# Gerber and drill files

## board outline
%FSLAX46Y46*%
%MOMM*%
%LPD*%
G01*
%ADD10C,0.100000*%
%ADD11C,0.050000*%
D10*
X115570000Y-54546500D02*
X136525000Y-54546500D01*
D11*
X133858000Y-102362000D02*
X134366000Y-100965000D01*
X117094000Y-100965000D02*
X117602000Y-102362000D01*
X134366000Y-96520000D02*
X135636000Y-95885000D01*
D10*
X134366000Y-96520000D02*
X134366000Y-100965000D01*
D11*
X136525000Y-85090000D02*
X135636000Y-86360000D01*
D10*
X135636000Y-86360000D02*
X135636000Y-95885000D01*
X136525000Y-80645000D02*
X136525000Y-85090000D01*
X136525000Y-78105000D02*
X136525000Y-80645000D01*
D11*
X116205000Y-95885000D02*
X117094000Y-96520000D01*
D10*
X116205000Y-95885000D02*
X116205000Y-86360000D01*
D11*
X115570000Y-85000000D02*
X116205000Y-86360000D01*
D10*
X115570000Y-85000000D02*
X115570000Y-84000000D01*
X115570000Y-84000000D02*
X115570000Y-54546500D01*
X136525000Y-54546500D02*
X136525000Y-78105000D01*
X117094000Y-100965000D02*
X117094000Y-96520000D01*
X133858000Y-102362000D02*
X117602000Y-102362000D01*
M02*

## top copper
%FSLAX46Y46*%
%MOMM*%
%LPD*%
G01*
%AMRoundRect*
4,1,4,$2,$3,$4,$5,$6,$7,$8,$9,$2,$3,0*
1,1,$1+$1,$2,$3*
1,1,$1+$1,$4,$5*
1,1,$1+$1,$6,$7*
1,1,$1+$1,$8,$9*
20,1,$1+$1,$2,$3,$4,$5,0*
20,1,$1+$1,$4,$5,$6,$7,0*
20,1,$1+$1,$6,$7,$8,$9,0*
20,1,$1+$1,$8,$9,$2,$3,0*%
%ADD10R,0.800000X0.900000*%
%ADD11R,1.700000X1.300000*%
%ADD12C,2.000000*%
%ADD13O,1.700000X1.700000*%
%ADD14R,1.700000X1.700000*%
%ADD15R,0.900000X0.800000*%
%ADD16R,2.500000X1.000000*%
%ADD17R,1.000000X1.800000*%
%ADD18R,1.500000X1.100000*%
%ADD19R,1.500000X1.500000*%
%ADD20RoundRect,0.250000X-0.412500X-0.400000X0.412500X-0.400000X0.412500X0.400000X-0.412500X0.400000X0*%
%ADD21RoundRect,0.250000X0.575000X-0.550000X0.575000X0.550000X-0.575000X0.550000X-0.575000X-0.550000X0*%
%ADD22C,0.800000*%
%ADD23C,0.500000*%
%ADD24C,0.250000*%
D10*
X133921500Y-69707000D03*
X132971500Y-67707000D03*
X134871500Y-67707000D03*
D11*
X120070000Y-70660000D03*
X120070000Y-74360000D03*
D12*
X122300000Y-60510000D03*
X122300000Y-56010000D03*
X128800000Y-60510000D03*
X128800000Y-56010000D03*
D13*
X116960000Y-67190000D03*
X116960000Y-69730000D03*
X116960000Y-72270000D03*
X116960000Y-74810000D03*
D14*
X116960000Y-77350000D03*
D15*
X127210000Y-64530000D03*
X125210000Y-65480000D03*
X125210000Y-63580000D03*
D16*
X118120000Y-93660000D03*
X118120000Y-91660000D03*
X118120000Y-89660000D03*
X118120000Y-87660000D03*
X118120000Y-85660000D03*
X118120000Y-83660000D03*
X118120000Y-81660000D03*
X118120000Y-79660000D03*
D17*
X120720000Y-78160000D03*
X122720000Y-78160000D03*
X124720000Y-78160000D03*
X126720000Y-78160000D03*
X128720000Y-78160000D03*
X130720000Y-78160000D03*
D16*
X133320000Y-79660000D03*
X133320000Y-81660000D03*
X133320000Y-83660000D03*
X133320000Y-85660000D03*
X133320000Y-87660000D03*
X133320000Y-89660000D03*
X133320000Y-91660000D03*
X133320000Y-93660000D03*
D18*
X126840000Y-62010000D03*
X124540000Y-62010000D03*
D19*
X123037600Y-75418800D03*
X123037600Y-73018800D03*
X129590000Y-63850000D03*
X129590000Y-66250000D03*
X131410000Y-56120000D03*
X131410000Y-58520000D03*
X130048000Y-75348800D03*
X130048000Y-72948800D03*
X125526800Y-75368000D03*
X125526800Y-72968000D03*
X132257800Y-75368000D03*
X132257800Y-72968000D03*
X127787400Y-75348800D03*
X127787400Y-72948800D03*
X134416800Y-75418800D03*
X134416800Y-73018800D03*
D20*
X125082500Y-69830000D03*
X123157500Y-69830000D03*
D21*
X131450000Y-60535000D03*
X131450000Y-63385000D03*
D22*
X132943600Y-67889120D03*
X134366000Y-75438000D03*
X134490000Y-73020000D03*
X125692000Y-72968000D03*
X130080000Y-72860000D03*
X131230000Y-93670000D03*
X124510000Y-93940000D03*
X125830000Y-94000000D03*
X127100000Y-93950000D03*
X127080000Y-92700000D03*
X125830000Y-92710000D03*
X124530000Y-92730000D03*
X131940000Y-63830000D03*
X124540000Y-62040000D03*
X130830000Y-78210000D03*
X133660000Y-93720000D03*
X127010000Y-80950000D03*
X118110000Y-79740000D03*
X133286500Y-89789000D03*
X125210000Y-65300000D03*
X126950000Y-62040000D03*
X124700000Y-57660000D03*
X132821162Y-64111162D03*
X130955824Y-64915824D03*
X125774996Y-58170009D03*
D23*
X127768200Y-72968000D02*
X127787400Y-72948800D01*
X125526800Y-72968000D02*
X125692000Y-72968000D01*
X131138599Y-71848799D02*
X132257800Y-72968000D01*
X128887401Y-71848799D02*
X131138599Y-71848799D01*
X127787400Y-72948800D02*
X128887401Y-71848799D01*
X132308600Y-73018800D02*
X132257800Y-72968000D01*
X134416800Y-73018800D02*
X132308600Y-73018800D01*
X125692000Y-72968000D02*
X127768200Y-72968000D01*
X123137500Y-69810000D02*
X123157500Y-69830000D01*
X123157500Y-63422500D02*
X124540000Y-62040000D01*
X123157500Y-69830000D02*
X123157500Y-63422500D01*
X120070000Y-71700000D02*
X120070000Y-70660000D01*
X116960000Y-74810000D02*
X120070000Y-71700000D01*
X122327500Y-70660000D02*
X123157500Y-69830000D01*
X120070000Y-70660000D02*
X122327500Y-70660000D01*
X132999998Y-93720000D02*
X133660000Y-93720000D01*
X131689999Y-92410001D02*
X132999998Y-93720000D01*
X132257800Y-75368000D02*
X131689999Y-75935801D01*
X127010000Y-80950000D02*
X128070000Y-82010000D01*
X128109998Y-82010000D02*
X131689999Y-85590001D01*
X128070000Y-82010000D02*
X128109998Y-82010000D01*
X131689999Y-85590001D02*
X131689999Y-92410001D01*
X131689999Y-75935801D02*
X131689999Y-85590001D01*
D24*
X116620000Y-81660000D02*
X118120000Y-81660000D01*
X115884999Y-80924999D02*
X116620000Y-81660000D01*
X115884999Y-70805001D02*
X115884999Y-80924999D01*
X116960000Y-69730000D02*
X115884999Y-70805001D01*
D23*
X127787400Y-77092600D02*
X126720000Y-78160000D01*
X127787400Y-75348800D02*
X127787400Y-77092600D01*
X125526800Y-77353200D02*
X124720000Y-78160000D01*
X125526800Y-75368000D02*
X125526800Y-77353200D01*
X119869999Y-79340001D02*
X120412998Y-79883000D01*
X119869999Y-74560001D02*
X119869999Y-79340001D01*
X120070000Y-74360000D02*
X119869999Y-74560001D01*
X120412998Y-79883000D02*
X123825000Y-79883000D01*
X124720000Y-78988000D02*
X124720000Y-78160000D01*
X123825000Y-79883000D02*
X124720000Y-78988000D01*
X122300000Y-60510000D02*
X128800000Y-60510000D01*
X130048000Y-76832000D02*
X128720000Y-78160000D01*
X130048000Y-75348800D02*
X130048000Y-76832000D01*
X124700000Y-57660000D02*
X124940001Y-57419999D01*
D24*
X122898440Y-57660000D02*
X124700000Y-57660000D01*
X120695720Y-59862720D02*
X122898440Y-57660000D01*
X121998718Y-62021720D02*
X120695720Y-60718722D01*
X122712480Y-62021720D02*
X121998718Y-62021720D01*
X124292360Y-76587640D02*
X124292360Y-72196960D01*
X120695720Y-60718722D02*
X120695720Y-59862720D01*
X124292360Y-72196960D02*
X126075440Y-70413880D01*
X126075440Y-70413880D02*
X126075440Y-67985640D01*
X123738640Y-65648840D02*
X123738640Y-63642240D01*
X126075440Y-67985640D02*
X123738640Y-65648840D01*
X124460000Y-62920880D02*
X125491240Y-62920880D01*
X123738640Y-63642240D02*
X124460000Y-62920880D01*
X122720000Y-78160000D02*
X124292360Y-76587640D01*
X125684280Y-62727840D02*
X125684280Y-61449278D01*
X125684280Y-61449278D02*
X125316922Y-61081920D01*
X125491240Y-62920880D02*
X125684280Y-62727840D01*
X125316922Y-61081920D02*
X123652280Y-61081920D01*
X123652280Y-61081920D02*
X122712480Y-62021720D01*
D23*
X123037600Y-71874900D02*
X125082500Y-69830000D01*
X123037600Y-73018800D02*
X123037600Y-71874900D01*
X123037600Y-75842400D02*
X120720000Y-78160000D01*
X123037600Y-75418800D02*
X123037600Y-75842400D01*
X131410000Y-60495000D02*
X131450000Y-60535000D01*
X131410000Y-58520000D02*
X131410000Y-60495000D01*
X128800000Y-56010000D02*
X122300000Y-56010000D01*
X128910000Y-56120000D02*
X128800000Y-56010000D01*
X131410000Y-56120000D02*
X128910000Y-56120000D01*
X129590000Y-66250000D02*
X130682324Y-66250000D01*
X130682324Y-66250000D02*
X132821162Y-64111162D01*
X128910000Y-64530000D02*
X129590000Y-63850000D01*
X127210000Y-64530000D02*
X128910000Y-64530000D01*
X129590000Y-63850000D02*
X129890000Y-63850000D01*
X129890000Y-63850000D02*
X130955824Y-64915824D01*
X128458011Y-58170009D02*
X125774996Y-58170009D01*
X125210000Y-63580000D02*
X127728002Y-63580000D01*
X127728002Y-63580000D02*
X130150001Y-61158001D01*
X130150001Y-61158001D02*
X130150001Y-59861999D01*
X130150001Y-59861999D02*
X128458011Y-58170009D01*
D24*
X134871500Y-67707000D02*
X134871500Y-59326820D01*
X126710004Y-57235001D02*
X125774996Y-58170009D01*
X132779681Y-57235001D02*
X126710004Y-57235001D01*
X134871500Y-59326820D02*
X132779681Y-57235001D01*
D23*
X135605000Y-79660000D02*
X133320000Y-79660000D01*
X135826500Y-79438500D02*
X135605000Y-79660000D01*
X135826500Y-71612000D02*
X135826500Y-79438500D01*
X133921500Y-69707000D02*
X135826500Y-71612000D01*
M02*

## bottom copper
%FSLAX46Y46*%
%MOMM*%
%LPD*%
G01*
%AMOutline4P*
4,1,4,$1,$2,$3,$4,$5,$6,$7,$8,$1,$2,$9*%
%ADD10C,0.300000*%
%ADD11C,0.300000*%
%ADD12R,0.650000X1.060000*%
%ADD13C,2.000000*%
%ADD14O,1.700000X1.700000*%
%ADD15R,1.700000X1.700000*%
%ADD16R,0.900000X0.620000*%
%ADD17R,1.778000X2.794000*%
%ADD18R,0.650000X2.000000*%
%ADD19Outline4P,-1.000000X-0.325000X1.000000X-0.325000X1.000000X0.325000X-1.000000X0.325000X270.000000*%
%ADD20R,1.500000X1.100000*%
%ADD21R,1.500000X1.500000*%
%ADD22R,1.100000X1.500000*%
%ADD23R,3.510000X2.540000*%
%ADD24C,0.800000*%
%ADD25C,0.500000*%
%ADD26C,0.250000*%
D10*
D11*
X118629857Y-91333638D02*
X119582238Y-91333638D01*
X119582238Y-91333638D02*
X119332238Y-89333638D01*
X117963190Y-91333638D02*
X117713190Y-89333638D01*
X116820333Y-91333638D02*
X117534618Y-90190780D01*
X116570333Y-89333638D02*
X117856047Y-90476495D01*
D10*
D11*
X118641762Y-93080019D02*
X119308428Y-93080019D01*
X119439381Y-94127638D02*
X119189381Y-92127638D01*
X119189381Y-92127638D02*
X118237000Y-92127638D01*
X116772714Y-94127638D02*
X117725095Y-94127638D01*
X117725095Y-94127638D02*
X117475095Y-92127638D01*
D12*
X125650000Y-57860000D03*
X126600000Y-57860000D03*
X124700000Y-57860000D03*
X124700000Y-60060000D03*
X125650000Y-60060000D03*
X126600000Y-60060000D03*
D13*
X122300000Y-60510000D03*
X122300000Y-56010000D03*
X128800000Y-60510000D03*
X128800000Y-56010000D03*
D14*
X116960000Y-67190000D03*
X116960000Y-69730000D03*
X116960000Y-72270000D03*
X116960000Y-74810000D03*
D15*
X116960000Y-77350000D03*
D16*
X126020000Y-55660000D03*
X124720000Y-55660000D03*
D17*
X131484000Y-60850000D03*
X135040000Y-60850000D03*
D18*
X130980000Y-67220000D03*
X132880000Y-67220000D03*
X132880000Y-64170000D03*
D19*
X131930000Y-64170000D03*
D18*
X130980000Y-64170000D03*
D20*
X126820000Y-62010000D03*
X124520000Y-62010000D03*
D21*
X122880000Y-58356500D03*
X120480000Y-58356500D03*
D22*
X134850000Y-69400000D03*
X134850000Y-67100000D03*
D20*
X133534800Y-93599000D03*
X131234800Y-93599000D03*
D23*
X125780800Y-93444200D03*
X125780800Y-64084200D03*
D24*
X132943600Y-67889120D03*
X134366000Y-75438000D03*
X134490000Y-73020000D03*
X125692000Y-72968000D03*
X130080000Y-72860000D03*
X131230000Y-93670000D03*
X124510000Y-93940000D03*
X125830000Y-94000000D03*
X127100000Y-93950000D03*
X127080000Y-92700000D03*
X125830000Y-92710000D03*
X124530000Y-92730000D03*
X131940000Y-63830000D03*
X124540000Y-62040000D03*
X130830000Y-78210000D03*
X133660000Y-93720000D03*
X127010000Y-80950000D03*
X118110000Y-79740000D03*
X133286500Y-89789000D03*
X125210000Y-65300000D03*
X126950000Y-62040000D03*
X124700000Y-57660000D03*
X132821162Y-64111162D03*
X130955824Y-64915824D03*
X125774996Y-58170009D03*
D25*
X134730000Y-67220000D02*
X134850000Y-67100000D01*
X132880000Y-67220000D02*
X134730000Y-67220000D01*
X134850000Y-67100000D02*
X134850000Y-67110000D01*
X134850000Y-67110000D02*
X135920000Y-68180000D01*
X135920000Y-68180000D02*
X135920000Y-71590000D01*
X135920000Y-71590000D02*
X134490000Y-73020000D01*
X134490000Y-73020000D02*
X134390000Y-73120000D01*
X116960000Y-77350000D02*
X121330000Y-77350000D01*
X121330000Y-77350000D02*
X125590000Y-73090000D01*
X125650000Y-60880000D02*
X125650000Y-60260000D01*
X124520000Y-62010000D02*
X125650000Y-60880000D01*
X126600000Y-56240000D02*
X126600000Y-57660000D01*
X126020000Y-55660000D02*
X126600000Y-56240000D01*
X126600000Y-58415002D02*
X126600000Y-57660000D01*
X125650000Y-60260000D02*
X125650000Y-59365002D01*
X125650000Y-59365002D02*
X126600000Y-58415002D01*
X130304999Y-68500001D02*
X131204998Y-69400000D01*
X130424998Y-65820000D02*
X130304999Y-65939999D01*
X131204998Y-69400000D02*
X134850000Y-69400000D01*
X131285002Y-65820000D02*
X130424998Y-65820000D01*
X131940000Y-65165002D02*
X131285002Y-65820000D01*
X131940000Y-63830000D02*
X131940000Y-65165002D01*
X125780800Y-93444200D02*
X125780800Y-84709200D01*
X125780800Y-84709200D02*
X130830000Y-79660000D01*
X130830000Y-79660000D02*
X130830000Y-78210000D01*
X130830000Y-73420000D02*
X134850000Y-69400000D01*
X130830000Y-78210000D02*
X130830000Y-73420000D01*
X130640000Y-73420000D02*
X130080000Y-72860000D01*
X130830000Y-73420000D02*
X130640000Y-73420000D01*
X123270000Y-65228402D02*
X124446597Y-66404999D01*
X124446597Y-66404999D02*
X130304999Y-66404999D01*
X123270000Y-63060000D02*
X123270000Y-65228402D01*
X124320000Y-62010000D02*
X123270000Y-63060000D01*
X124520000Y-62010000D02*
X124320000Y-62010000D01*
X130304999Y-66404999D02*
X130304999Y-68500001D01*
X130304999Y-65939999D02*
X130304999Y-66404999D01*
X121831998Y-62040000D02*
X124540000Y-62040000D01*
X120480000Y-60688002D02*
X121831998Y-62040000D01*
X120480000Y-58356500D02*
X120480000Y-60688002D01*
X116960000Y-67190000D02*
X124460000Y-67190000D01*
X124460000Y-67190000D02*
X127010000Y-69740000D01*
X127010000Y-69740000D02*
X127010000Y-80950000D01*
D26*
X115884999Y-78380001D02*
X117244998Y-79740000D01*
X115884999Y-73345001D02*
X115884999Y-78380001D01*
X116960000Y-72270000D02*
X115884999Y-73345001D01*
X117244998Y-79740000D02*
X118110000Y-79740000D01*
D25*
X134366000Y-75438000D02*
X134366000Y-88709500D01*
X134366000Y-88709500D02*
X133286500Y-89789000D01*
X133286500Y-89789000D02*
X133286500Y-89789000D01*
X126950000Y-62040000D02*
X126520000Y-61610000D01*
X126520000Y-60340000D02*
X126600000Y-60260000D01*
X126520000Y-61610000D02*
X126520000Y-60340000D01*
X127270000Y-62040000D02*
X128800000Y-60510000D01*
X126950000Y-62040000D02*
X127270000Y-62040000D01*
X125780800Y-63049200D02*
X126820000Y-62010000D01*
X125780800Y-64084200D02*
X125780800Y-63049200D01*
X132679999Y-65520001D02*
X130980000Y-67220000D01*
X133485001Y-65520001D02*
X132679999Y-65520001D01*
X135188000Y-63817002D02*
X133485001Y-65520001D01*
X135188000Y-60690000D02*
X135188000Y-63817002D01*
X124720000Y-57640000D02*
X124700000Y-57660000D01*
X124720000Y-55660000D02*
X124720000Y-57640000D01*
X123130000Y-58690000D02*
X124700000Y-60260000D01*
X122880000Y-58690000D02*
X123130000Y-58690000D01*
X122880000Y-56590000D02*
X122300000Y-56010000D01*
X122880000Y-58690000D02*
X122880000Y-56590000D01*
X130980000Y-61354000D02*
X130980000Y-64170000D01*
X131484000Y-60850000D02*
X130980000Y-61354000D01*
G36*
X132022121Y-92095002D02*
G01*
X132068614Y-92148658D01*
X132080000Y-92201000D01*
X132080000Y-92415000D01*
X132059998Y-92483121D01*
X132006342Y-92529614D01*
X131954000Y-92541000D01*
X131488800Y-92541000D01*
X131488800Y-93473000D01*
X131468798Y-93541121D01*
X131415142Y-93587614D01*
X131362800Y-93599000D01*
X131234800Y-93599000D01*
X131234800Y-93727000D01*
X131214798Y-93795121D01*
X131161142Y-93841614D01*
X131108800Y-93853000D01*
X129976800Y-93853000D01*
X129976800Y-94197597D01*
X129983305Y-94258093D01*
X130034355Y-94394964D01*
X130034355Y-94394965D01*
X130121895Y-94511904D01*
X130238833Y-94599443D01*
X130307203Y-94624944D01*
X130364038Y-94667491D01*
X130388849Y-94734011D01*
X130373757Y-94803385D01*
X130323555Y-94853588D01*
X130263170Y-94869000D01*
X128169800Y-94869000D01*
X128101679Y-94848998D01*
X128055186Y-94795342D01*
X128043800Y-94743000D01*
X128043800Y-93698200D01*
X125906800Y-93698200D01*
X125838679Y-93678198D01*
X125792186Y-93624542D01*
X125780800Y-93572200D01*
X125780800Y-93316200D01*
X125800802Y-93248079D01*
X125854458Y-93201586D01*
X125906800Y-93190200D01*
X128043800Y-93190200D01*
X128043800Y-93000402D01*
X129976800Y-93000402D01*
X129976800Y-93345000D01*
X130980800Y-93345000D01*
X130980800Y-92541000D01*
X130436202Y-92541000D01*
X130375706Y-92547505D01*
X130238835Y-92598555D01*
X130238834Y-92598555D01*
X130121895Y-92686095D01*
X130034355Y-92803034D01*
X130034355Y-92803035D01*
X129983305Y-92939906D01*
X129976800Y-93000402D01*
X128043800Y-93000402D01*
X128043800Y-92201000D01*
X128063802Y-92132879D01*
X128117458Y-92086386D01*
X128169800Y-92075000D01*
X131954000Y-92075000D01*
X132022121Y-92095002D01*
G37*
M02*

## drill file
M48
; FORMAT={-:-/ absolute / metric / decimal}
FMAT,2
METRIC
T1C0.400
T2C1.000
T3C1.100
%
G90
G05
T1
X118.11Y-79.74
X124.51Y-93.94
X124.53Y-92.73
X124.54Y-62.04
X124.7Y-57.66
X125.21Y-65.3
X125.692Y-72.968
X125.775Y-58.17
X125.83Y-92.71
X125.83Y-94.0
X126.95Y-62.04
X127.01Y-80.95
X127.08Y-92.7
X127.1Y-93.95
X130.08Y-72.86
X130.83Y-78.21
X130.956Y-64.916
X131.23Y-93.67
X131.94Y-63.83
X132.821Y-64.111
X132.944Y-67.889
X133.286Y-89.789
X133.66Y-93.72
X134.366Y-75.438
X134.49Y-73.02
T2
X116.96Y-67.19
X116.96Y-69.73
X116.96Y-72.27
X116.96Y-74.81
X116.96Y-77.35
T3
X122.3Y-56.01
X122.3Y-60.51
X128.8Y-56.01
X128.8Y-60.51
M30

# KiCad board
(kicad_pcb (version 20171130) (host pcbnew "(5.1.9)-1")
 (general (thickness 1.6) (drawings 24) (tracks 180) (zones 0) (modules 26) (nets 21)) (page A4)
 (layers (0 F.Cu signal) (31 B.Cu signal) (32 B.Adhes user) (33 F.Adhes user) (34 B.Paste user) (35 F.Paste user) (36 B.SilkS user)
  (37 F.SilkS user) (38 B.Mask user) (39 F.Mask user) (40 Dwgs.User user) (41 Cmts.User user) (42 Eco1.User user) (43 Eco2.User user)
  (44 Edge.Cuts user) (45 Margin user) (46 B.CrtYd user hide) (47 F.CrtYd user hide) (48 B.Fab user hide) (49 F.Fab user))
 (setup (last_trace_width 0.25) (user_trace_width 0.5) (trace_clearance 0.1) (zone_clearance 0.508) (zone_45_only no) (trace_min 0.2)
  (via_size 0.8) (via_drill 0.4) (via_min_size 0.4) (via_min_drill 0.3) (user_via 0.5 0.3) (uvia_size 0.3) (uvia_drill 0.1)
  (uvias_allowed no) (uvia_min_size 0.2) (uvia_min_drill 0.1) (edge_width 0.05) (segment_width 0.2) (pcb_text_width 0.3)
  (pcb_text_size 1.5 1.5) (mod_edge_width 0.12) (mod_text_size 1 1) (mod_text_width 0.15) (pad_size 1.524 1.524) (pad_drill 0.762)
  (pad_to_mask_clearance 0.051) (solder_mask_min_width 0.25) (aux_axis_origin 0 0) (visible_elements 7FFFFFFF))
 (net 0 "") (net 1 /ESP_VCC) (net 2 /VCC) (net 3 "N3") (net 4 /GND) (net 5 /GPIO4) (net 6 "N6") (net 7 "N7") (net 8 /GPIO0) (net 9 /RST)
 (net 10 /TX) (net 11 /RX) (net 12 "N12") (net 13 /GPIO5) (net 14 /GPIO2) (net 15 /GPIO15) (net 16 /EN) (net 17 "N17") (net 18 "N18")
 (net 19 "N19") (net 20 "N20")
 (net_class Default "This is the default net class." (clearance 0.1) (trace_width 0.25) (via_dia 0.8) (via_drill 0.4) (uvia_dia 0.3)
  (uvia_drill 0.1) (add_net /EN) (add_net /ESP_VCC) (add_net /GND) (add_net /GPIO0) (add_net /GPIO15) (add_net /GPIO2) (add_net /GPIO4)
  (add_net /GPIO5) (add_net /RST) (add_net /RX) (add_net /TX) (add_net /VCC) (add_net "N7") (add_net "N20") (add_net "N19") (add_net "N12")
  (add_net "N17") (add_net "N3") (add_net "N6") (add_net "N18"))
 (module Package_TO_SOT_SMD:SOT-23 (layer F.Cu) (at 133.9215 68.707 270)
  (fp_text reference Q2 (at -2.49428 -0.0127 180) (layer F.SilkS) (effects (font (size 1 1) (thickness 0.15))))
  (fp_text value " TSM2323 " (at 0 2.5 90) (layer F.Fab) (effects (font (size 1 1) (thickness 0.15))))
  (pad 3 smd rect (at 1 0 270) (size 0.9 0.8) (layers F.Cu F.Paste F.Mask) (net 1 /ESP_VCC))
  (pad 2 smd rect (at -1 0.95 270) (size 0.9 0.8) (layers F.Cu F.Paste F.Mask) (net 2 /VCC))
  (pad 1 smd rect (at -1 -0.95 270) (size 0.9 0.8) (layers F.Cu F.Paste F.Mask) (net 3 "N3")))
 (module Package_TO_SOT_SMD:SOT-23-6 (layer B.Cu) (at 125.65 58.96 90)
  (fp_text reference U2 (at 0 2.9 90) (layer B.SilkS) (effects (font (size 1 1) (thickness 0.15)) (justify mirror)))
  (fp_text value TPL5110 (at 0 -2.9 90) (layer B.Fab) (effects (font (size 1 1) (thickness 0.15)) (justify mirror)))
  (pad 5 smd rect (at 1.1 0 90) (size 1.06 0.65) (layers B.Cu B.Paste B.Mask) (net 3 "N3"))
  (pad 6 smd rect (at 1.1 0.95 90) (size 1.06 0.65) (layers B.Cu B.Paste B.Mask) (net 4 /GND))
  (pad 4 smd rect (at 1.1 -0.95 90) (size 1.06 0.65) (layers B.Cu B.Paste B.Mask) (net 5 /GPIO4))
  (pad 3 smd rect (at -1.1 -0.95 90) (size 1.06 0.65) (layers B.Cu B.Paste B.Mask) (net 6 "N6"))
  (pad 2 smd rect (at -1.1 0 90) (size 1.06 0.65) (layers B.Cu B.Paste B.Mask) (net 4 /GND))
  (pad 1 smd rect (at -1.1 0.95 90) (size 1.06 0.65) (layers B.Cu B.Paste B.Mask) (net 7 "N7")))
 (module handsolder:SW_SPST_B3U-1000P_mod (layer F.Cu) (at 120.07 72.51 90)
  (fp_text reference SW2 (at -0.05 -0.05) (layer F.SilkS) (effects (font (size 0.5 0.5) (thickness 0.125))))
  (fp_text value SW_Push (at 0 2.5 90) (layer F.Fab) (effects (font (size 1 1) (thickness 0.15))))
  (pad 2 smd rect (at 1.85 0 90) (size 1.3 1.7) (layers F.Cu F.Paste F.Mask) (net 4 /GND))
  (pad 1 smd rect (at -1.85 0 90) (size 1.3 1.7) (layers F.Cu F.Paste F.Mask) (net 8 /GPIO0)))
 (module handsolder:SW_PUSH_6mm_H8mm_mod (layer F.Cu) (at 128.8 60.51 180)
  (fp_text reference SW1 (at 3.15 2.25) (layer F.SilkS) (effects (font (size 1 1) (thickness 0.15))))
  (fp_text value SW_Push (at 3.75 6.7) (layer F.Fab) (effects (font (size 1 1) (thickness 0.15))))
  (pad 1 thru_hole circle (at 6.5 0 270) (size 2 2) (drill 1.1) (layers *.Cu *.Mask) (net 7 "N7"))
  (pad 2 thru_hole circle (at 6.5 4.5 270) (size 2 2) (drill 1.1) (layers *.Cu *.Mask) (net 6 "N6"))
  (pad 1 thru_hole circle (at 0 0 270) (size 2 2) (drill 1.1) (layers *.Cu *.Mask) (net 7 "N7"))
  (pad 2 thru_hole circle (at 0 4.5 270) (size 2 2) (drill 1.1) (layers *.Cu *.Mask) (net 6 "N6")))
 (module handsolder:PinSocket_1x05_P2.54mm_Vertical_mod (layer F.Cu) (at 116.96 77.35 180)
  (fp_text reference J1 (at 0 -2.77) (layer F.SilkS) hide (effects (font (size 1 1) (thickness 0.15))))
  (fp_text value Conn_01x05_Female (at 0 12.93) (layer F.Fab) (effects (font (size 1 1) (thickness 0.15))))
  (pad 5 thru_hole oval (at 0 10.16 180) (size 1.7 1.7) (drill 1) (layers *.Cu *.Mask) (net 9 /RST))
  (pad 4 thru_hole oval (at 0 7.62 180) (size 1.7 1.7) (drill 1) (layers *.Cu *.Mask) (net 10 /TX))
  (pad 3 thru_hole oval (at 0 5.08 180) (size 1.7 1.7) (drill 1) (layers *.Cu *.Mask) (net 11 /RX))
  (pad 2 thru_hole oval (at 0 2.54 180) (size 1.7 1.7) (drill 1) (layers *.Cu *.Mask) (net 4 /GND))
  (pad 1 thru_hole rect (at 0 0 180) (size 1.7 1.7) (drill 1) (layers *.Cu *.Mask) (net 2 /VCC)))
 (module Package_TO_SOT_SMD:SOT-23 (layer F.Cu) (at 126.21 64.53)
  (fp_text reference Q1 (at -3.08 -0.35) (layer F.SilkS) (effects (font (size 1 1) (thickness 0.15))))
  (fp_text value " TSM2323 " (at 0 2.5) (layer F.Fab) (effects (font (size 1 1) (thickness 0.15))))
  (pad 3 smd rect (at 1 0) (size 0.9 0.8) (layers F.Cu F.Paste F.Mask) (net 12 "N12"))
  (pad 2 smd rect (at -1 0.95) (size 0.9 0.8) (layers F.Cu F.Paste F.Mask) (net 7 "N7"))
  (pad 1 smd rect (at -1 -0.95) (size 0.9 0.8) (layers F.Cu F.Paste F.Mask) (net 3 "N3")))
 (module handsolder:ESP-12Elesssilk (layer F.Cu) (at 125.72 90.16 180)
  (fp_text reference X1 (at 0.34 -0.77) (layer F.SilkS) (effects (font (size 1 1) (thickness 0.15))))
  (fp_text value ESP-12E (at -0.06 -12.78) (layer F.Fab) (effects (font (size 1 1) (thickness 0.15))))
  (pad 22 smd rect (at 7.6 -3.5 180) (size 2.5 1) (layers F.Cu F.Paste F.Mask))
  (pad 21 smd rect (at 7.6 -1.5 180) (size 2.5 1) (layers F.Cu F.Paste F.Mask))
  (pad 20 smd rect (at 7.6 0.5 180) (size 2.5 1) (layers F.Cu F.Paste F.Mask))
  (pad 19 smd rect (at 7.6 2.5 180) (size 2.5 1) (layers F.Cu F.Paste F.Mask))
  (pad 18 smd rect (at 7.6 4.5 180) (size 2.5 1) (layers F.Cu F.Paste F.Mask))
  (pad 17 smd rect (at 7.6 6.5 180) (size 2.5 1) (layers F.Cu F.Paste F.Mask))
  (pad 16 smd rect (at 7.6 8.5 180) (size 2.5 1) (layers F.Cu F.Paste F.Mask) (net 10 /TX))
  (pad 15 smd rect (at 7.6 10.5 180) (size 2.5 1) (layers F.Cu F.Paste F.Mask) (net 11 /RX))
  (pad 14 smd rect (at 5 12 180) (size 1 1.8) (layers F.Cu F.Paste F.Mask) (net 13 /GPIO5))
  (pad 13 smd rect (at 3 12 180) (size 1 1.8) (layers F.Cu F.Paste F.Mask) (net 5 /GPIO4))
  (pad 12 smd rect (at 1 12 180) (size 1 1.8) (layers F.Cu F.Paste F.Mask) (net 8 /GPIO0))
  (pad 11 smd rect (at -1 12 180) (size 1 1.8) (layers F.Cu F.Paste F.Mask) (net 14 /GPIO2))
  (pad 10 smd rect (at -3 12 180) (size 1 1.8) (layers F.Cu F.Paste F.Mask) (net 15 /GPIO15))
  (pad 9 smd rect (at -5 12 180) (size 1 1.8) (layers F.Cu F.Paste F.Mask) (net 4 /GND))
  (pad 8 smd rect (at -7.6 10.5 180) (size 2.5 1) (layers F.Cu F.Paste F.Mask) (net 1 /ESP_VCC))
  (pad 7 smd rect (at -7.6 8.5 180) (size 2.5 1) (layers F.Cu F.Paste F.Mask))
  (pad 6 smd rect (at -7.6 6.5 180) (size 2.5 1) (layers F.Cu F.Paste F.Mask))
  (pad 5 smd rect (at -7.6 4.5 180) (size 2.5 1) (layers F.Cu F.Paste F.Mask))
  (pad 4 smd rect (at -7.6 2.5 180) (size 2.5 1) (layers F.Cu F.Paste F.Mask))
  (pad 3 smd rect (at -7.6 0.5 180) (size 2.5 1) (layers F.Cu F.Paste F.Mask) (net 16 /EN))
  (pad 2 smd rect (at -7.6 -1.5 180) (size 2.5 1) (layers F.Cu F.Paste F.Mask))
  (pad 1 smd rect (at -7.6 -3.5 180) (size 2.5 1) (layers F.Cu F.Paste F.Mask) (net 9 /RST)))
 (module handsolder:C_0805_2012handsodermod (layer F.Cu) (at 125.69 62.01)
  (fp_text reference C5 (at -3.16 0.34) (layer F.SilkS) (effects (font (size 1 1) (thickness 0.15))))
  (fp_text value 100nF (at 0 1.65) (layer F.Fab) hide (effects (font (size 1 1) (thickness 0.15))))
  (pad 2 smd rect (at 1.15 0) (size 1.5 1.1) (layers F.Cu F.Paste F.Mask) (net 7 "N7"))
  (pad 1 smd rect (at -1.15 0) (size 1.5 1.1) (layers F.Cu F.Paste F.Mask) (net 4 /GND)))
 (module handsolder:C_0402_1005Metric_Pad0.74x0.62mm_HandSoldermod (layer B.Cu) (at 125.37 55.66)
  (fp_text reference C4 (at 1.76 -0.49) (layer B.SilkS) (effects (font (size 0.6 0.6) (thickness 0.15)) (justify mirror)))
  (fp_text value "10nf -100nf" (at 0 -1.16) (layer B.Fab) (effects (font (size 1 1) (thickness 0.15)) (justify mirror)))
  (pad 2 smd rect (at 0.65 0) (size 0.9 0.62) (layers B.Cu B.Paste B.Mask) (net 4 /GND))
  (pad 1 smd rect (at -0.65 0) (size 0.9 0.62) (layers B.Cu B.Paste B.Mask) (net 5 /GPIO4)))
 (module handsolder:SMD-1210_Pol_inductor (layer B.Cu) (at 133.262 60.85)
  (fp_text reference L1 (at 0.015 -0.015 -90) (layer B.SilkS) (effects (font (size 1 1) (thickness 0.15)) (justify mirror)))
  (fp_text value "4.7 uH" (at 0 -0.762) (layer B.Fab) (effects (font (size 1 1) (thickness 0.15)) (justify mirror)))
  (pad 1 smd rect (at -1.778 0) (size 1.778 2.794) (layers B.Cu B.Paste B.Mask) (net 12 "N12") (zone_connect 2))
  (pad 2 smd rect (at 1.778 0) (size 1.778 2.794) (layers B.Cu B.Paste B.Mask) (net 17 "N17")))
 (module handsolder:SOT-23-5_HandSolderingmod (layer B.Cu) (at 131.93 65.72 270)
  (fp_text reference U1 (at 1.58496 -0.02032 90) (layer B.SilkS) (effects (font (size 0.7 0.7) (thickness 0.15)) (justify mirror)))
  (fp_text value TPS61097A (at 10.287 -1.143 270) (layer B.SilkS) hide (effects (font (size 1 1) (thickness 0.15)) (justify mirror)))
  (pad 5 smd rect (at 1.5 0.95 270) (size 2 0.65) (layers B.Cu B.Paste B.Mask) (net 17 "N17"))
  (pad 4 smd rect (at 1.5 -0.95 270) (size 2 0.65) (layers B.Cu B.Paste B.Mask) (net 2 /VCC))
  (pad 3 smd rect (at -1.55 -0.95 270) (size 2 0.65) (layers B.Cu B.Paste B.Mask) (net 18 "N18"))
  (pad 2 smd trapezoid (at -1.55 0 270) (size 2 0.65) (layers B.Cu B.Paste B.Mask) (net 4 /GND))
  (pad 1 smd rect (at -1.55 0.95 270) (size 2 0.65) (layers B.Cu B.Paste B.Mask) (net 12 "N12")))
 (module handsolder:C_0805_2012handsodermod (layer B.Cu) (at 125.67 62.01)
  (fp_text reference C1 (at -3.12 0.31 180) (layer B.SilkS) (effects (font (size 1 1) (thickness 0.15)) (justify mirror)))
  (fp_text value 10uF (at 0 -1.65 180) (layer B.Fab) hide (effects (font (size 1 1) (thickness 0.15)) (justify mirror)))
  (pad 2 smd rect (at 1.15 0) (size 1.5 1.1) (layers B.Cu B.Paste B.Mask) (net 7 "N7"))
  (pad 1 smd rect (at -1.15 0) (size 1.5 1.1) (layers B.Cu B.Paste B.Mask) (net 4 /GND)))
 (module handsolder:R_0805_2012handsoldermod (layer F.Cu) (at 123.0376 74.2188 270)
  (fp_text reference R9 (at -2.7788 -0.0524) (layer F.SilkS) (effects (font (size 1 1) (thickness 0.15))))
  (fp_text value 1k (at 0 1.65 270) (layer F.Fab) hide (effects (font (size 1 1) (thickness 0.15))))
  (pad 2 smd rect (at 1.2 0 270) (size 1.5 1.5) (layers F.Cu F.Paste F.Mask) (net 13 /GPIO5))
  (pad 1 smd rect (at -1.2 0 270) (size 1.5 1.5) (layers F.Cu F.Paste F.Mask) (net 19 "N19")))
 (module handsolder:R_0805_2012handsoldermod (layer B.Cu) (at 121.68 58.3565)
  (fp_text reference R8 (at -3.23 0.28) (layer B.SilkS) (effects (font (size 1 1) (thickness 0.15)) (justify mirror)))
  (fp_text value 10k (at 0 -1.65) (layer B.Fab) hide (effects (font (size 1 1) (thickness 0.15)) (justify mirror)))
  (pad 2 smd rect (at 1.2 0) (size 1.5 1.5) (layers B.Cu B.Paste B.Mask) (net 6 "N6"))
  (pad 1 smd rect (at -1.2 0) (size 1.5 1.5) (layers B.Cu B.Paste B.Mask) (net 4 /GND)))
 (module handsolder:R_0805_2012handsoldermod (layer F.Cu) (at 129.59 65.05 90)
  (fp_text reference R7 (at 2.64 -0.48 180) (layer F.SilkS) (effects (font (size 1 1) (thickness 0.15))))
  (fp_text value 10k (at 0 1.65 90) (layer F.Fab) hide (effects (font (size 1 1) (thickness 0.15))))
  (pad 2 smd rect (at 1.2 0 90) (size 1.5 1.5) (layers F.Cu F.Paste F.Mask) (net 12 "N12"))
  (pad 1 smd rect (at -1.2 0 90) (size 1.5 1.5) (layers F.Cu F.Paste F.Mask) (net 18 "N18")))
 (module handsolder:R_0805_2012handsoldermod (layer F.Cu) (at 131.41 57.32 90)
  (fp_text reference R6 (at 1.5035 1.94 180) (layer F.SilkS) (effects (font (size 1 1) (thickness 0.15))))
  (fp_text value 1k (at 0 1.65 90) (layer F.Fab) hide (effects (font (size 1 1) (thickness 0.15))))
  (pad 2 smd rect (at 1.2 0 90) (size 1.5 1.5) (layers F.Cu F.Paste F.Mask) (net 6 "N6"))
  (pad 1 smd rect (at -1.2 0 90) (size 1.5 1.5) (layers F.Cu F.Paste F.Mask) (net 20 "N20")))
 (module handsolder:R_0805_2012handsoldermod (layer F.Cu) (at 130.048 74.1488 270)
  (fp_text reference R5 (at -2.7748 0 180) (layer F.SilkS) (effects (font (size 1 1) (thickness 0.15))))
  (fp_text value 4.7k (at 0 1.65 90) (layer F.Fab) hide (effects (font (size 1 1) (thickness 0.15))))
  (pad 2 smd rect (at 1.2 0 270) (size 1.5 1.5) (layers F.Cu F.Paste F.Mask) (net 15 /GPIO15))
  (pad 1 smd rect (at -1.2 0 270) (size 1.5 1.5) (layers F.Cu F.Paste F.Mask) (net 4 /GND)))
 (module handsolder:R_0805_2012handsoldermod (layer F.Cu) (at 125.5268 74.168 270)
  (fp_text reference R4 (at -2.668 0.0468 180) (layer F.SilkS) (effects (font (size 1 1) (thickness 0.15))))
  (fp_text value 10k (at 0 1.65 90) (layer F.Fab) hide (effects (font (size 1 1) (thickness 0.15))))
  (pad 2 smd rect (at 1.2 0 270) (size 1.5 1.5) (layers F.Cu F.Paste F.Mask) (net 8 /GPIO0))
  (pad 1 smd rect (at -1.2 0 270) (size 1.5 1.5) (layers F.Cu F.Paste F.Mask) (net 2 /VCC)))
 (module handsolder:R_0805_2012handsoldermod (layer F.Cu) (at 132.2578 74.168 270)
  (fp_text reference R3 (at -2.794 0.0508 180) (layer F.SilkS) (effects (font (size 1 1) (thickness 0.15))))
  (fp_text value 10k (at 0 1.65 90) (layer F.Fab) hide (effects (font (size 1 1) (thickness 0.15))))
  (pad 2 smd rect (at 1.2 0 270) (size 1.5 1.5) (layers F.Cu F.Paste F.Mask) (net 9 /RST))
  (pad 1 smd rect (at -1.2 0 270) (size 1.5 1.5) (layers F.Cu F.Paste F.Mask) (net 2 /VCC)))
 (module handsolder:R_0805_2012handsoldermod (layer F.Cu) (at 127.7874 74.1488 270)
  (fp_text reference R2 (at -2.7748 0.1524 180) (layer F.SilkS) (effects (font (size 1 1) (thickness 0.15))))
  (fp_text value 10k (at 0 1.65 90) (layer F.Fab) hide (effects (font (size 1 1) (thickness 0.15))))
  (pad 2 smd rect (at 1.2 0 270) (size 1.5 1.5) (layers F.Cu F.Paste F.Mask) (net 14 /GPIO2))
  (pad 1 smd rect (at -1.2 0 270) (size 1.5 1.5) (layers F.Cu F.Paste F.Mask) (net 2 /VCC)))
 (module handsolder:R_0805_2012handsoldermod (layer F.Cu) (at 134.4168 74.2188 270)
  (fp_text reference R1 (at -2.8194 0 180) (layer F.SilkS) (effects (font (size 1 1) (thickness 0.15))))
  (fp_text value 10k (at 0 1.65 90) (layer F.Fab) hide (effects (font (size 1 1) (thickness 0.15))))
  (pad 2 smd rect (at 1.2 0 270) (size 1.5 1.5) (layers F.Cu F.Paste F.Mask) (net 16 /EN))
  (pad 1 smd rect (at -1.2 0 270) (size 1.5 1.5) (layers F.Cu F.Paste F.Mask) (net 2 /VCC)))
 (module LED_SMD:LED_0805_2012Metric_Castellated (layer F.Cu) (at 124.12 69.83)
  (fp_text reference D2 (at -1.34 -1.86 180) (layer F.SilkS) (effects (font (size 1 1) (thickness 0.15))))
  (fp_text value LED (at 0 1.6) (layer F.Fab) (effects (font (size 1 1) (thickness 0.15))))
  (pad 2 smd roundrect (at 0.9625 0) (size 1.325 1.3) (layers F.Cu F.Paste F.Mask) (roundrect_rratio 0.1923076923076923) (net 19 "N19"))
  (pad 1 smd roundrect (at -0.9625 0) (size 1.325 1.3) (layers F.Cu F.Paste F.Mask) (roundrect_rratio 0.1923076923076923) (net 4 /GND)))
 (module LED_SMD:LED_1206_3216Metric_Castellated (layer F.Cu) (at 131.45 61.96 90)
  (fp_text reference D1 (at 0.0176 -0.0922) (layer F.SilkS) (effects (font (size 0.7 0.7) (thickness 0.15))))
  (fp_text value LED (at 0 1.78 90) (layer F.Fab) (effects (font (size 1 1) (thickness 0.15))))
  (pad 2 smd roundrect (at 1.425 0 90) (size 1.6 1.65) (layers F.Cu F.Paste F.Mask) (roundrect_rratio 0.15625) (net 20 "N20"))
  (pad 1 smd roundrect (at -1.425 0 90) (size 1.6 1.65) (layers F.Cu F.Paste F.Mask) (roundrect_rratio 0.15625) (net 4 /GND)))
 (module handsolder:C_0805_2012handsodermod (layer B.Cu) (at 134.85 68.25 270)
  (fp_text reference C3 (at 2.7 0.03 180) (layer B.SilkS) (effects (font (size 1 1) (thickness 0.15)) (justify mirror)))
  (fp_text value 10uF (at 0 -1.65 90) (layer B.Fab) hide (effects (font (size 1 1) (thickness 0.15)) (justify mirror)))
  (pad 2 smd rect (at 1.15 0 270) (size 1.5 1.1) (layers B.Cu B.Paste B.Mask) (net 4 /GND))
  (pad 1 smd rect (at -1.15 0 270) (size 1.5 1.1) (layers B.Cu B.Paste B.Mask) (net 2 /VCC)))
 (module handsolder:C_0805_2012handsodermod (layer B.Cu) (at 132.3848 93.599)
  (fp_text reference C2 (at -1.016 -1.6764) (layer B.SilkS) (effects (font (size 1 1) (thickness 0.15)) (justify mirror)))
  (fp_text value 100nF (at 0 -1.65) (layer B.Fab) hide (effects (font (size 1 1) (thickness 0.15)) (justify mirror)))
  (pad 2 smd rect (at 1.15 0) (size 1.5 1.1) (layers B.Cu B.Paste B.Mask) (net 9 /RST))
  (pad 1 smd rect (at -1.15 0) (size 1.5 1.1) (layers B.Cu B.Paste B.Mask) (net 4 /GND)))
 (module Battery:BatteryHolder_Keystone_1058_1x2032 (layer B.Cu) (at 125.7808 78.7642 270)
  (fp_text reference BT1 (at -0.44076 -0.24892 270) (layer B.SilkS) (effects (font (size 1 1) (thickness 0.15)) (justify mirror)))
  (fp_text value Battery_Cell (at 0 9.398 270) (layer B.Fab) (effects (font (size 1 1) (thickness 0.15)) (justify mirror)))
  (pad 2 smd rect (at 14.68 0 270) (size 2.54 3.51) (layers B.Cu B.Paste B.Mask) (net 4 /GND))
  (pad 1 smd rect (at -14.68 0 270) (size 2.54 3.51) (layers B.Cu B.Paste B.Mask) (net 7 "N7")))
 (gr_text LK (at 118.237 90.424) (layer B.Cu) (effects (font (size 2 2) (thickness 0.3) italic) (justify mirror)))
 (gr_line (start 115.57 54.5465) (end 136.525 54.5465) (layer Edge.Cuts) (width 0.1))
 (gr_line (start 133.858 102.362) (end 134.366 100.965) (layer Edge.Cuts) (width 0.05))
 (gr_line (start 117.094 100.965) (end 117.602 102.362) (layer Edge.Cuts) (width 0.05))
 (gr_line (start 134.366 96.52) (end 135.636 95.885) (layer Edge.Cuts) (width 0.05))
 (gr_line (start 134.366 96.52) (end 134.366 100.965) (layer Edge.Cuts) (width 0.1))
 (gr_line (start 136.525 85.09) (end 135.636 86.36) (layer Edge.Cuts) (width 0.05))
 (gr_line (start 135.636 86.36) (end 135.636 95.885) (layer Edge.Cuts) (width 0.1))
 (gr_line (start 136.525 80.645) (end 136.525 85.09) (layer Edge.Cuts) (width 0.1))
 (gr_line (start 136.525 78.105) (end 136.525 80.645) (layer Edge.Cuts) (width 0.1))
 (gr_line (start 116.205 95.885) (end 117.094 96.52) (layer Edge.Cuts) (width 0.05))
 (gr_line (start 116.205 95.885) (end 116.205 86.36) (layer Edge.Cuts) (width 0.1))
 (gr_line (start 115.57 85) (end 116.205 86.36) (layer Edge.Cuts) (width 0.05))
 (gr_line (start 115.57 85) (end 115.57 84) (layer Edge.Cuts) (width 0.1))
 (gr_line (start 115.57 84) (end 115.57 54.5465) (layer Edge.Cuts) (width 0.1))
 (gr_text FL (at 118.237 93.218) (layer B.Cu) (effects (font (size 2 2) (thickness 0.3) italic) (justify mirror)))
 (gr_line (start 136.525 54.5465) (end 136.525 78.105) (layer Edge.Cuts) (width 0.1))
 (gr_line (start 117.094 100.965) (end 117.094 96.52) (layer Edge.Cuts) (width 0.1))
 (gr_line (start 133.858 102.362) (end 117.602 102.362) (layer Edge.Cuts) (width 0.1))
 (via (at 132.9436 67.88912) (size 0.8) (drill 0.4) (layers F.Cu B.Cu) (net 2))
 (via (at 134.366 75.438) (size 0.8) (drill 0.4) (layers F.Cu B.Cu) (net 16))
 (segment (start 134.73 67.22) (end 134.85 67.1) (width 0.5) (layer B.Cu) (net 2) (status 30))
 (segment (start 132.88 67.22) (end 134.73 67.22) (width 0.5) (layer B.Cu) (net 2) (status 30))
 (segment (start 127.7682 72.968) (end 127.7874 72.9488) (width 0.5) (layer F.Cu) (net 2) (status 30))
 (segment (start 125.5268 72.968) (end 125.692 72.968) (width 0.5) (layer F.Cu) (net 2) (status 30))
 (segment (start 131.138599 71.848799) (end 132.2578 72.968) (width 0.5) (layer F.Cu) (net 2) (status 20))
 (segment (start 128.887401 71.848799) (end 131.138599 71.848799) (width 0.5) (layer F.Cu) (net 2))
 (segment (start 127.7874 72.9488) (end 128.887401 71.848799) (width 0.5) (layer F.Cu) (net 2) (status 10))
 (segment (start 132.3086 73.0188) (end 132.2578 72.968) (width 0.5) (layer F.Cu) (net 2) (status 30))
 (segment (start 134.4168 73.0188) (end 132.3086 73.0188) (width 0.5) (layer F.Cu) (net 2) (status 30))
 (segment (start 134.85 67.1) (end 134.85 67.11) (width 0.5) (layer B.Cu) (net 2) (status 30))
 (segment (start 134.85 67.11) (end 135.92 68.18) (width 0.5) (layer B.Cu) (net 2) (status 10))
 (segment (start 135.92 68.18) (end 135.92 71.59) (width 0.5) (layer B.Cu) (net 2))
 (segment (start 135.92 71.59) (end 134.49 73.02) (width 0.5) (layer B.Cu) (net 2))
 (segment (start 134.49 73.02) (end 134.39 73.12) (width 0.5) (layer B.Cu) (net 2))
 (via (at 134.49 73.02) (size 0.8) (drill 0.4) (layers F.Cu B.Cu) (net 2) (status 30))
 (segment (start 116.96 77.35) (end 121.33 77.35) (width 0.5) (layer B.Cu) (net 2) (status 10))
 (segment (start 121.33 77.35) (end 125.59 73.09) (width 0.5) (layer B.Cu) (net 2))
 (segment (start 125.692 72.968) (end 127.7682 72.968) (width 0.5) (layer F.Cu) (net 2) (status 30))
 (via (at 125.692 72.968) (size 0.8) (drill 0.4) (layers F.Cu B.Cu) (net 2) (status 30))
 (via (at 130.08 72.86) (size 0.8) (drill 0.4) (layers F.Cu B.Cu) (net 4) (status 30))
 (via (at 131.23 93.67) (size 0.8) (drill 0.4) (layers F.Cu B.Cu) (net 4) (status 30))
 (via (at 124.51 93.94) (size 0.8) (drill 0.4) (layers F.Cu B.Cu) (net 4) (status 30))
 (via (at 125.83 94) (size 0.8) (drill 0.4) (layers F.Cu B.Cu) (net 4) (status 30))
 (via (at 127.1 93.95) (size 0.8) (drill 0.4) (layers F.Cu B.Cu) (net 4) (status 30))
 (via (at 127.08 92.7) (size 0.8) (drill 0.4) (layers F.Cu B.Cu) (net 4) (status 30))
 (via (at 125.83 92.71) (size 0.8) (drill 0.4) (layers F.Cu B.Cu) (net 4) (status 30))
 (via (at 124.53 92.73) (size 0.8) (drill 0.4) (layers F.Cu B.Cu) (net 4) (status 30))
 (via (at 131.94 63.83) (size 0.8) (drill 0.4) (layers F.Cu B.Cu) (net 4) (status 30))
 (via (at 124.54 62.04) (size 0.8) (drill 0.4) (layers F.Cu B.Cu) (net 4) (status 30))
 (segment (start 125.65 60.88) (end 125.65 60.26) (width 0.5) (layer B.Cu) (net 4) (status 20))
 (segment (start 124.52 62.01) (end 125.65 60.88) (width 0.5) (layer B.Cu) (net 4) (status 10))
 (segment (start 126.6 56.24) (end 126.6 57.66) (width 0.5) (layer B.Cu) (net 4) (status 20))
 (segment (start 126.02 55.66) (end 126.6 56.24) (width 0.5) (layer B.Cu) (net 4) (status 10))
 (segment (start 126.6 58.415002) (end 126.6 57.66) (width 0.5) (layer B.Cu) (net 4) (status 20))
 (segment (start 125.65 60.26) (end 125.65 59.365002) (width 0.5) (layer B.Cu) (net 4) (status 10))
 (segment (start 125.65 59.365002) (end 126.6 58.415002) (width 0.5) (layer B.Cu) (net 4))
 (segment (start 130.304999 68.500001) (end 131.204998 69.4) (width 0.5) (layer B.Cu) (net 4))
 (segment (start 130.424998 65.82) (end 130.304999 65.939999) (width 0.5) (layer B.Cu) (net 4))
 (segment (start 131.204998 69.4) (end 134.85 69.4) (width 0.5) (layer B.Cu) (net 4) (status 20))
 (segment (start 131.285002 65.82) (end 130.424998 65.82) (width 0.5) (layer B.Cu) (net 4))
 (segment (start 131.94 65.165002) (end 131.285002 65.82) (width 0.5) (layer B.Cu) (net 4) (status 10))
 (segment (start 131.94 63.83) (end 131.94 65.165002) (width 0.5) (layer B.Cu) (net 4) (status 30))
 (segment (start 125.7808 93.4442) (end 125.7808 84.7092) (width 0.5) (layer B.Cu) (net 4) (status 10))
 (segment (start 125.7808 84.7092) (end 130.83 79.66) (width 0.5) (layer B.Cu) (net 4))
 (segment (start 130.83 79.66) (end 130.83 78.21) (width 0.5) (layer B.Cu) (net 4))
 (via (at 130.83 78.21) (size 0.8) (drill 0.4) (layers F.Cu B.Cu) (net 4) (status 30))
 (segment (start 130.83 73.42) (end 134.85 69.4) (width 0.5) (layer B.Cu) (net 4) (status 20))
 (segment (start 130.83 78.21) (end 130.83 73.42) (width 0.5) (layer B.Cu) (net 4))
 (segment (start 130.64 73.42) (end 130.08 72.86) (width 0.5) (layer B.Cu) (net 4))
 (segment (start 130.83 73.42) (end 130.64 73.42) (width 0.5) (layer B.Cu) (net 4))
 (segment (start 123.1375 69.81) (end 123.1575 69.83) (width 0.5) (layer F.Cu) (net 4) (status 30))
 (segment (start 123.1575 63.4225) (end 124.54 62.04) (width 0.5) (layer F.Cu) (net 4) (status 20))
 (segment (start 123.1575 69.83) (end 123.1575 63.4225) (width 0.5) (layer F.Cu) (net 4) (status 10))
 (segment (start 123.27 65.228402) (end 124.446597 66.404999) (width 0.5) (layer B.Cu) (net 4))
 (segment (start 124.446597 66.404999) (end 130.304999 66.404999) (width 0.5) (layer B.Cu) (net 4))
 (segment (start 123.27 63.06) (end 123.27 65.228402) (width 0.5) (layer B.Cu) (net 4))
 (segment (start 124.32 62.01) (end 123.27 63.06) (width 0.5) (layer B.Cu) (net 4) (status 10))
 (segment (start 124.52 62.01) (end 124.32 62.01) (width 0.5) (layer B.Cu) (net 4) (status 30))
 (segment (start 130.304999 66.404999) (end 130.304999 68.500001) (width 0.5) (layer B.Cu) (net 4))
 (segment (start 130.304999 65.939999) (end 130.304999 66.404999) (width 0.5) (layer B.Cu) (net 4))
 (segment (start 120.07 71.7) (end 120.07 70.66) (width 0.5) (layer F.Cu) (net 4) (status 20))
 (segment (start 116.96 74.81) (end 120.07 71.7) (width 0.5) (layer F.Cu) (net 4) (status 10))
 (segment (start 122.3275 70.66) (end 123.1575 69.83) (width 0.5) (layer F.Cu) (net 4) (status 20))
 (segment (start 120.07 70.66) (end 122.3275 70.66) (width 0.5) (layer F.Cu) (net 4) (status 10))
 (segment (start 121.831998 62.04) (end 124.54 62.04) (width 0.5) (layer B.Cu) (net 4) (status 20))
 (segment (start 120.48 60.688002) (end 121.831998 62.04) (width 0.5) (layer B.Cu) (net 4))
 (segment (start 120.48 58.3565) (end 120.48 60.688002) (width 0.5) (layer B.Cu) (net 4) (status 10))
 (via (at 133.66 93.72) (size 0.8) (drill 0.4) (layers F.Cu B.Cu) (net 9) (status 30))
 (segment (start 132.999998 93.72) (end 133.66 93.72) (width 0.5) (layer F.Cu) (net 9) (status 30))
 (segment (start 131.689999 92.410001) (end 132.999998 93.72) (width 0.5) (layer F.Cu) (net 9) (status 20))
 (segment (start 132.2578 75.368) (end 131.689999 75.935801) (width 0.5) (layer F.Cu) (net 9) (status 30))
 (segment (start 116.96 67.19) (end 124.46 67.19) (width 0.5) (layer B.Cu) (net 9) (status 10))
 (segment (start 124.46 67.19) (end 127.01 69.74) (width 0.5) (layer B.Cu) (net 9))
 (segment (start 127.01 69.74) (end 127.01 80.95) (width 0.5) (layer B.Cu) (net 9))
 (via (at 127.01 80.95) (size 0.8) (drill 0.4) (layers F.Cu B.Cu) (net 9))
 (segment (start 127.01 80.95) (end 128.07 82.01) (width 0.5) (layer F.Cu) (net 9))
 (segment (start 128.109998 82.01) (end 131.689999 85.590001) (width 0.5) (layer F.Cu) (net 9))
 (segment (start 128.07 82.01) (end 128.109998 82.01) (width 0.5) (layer F.Cu) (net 9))
 (segment (start 131.689999 85.590001) (end 131.689999 92.410001) (width 0.5) (layer F.Cu) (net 9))
 (segment (start 131.689999 75.935801) (end 131.689999 85.590001) (width 0.5) (layer F.Cu) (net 9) (status 10))
 (segment (start 115.884999 78.380001) (end 117.244998 79.74) (width 0.25) (layer B.Cu) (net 11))
 (segment (start 115.884999 73.345001) (end 115.884999 78.380001) (width 0.25) (layer B.Cu) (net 11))
 (segment (start 116.96 72.27) (end 115.884999 73.345001) (width 0.25) (layer B.Cu) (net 11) (status 10))
 (segment (start 117.244998 79.74) (end 118.11 79.74) (width 0.25) (layer B.Cu) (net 11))
 (via (at 118.11 79.74) (size 0.8) (drill 0.4) (layers F.Cu B.Cu) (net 11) (status 30))
 (segment (start 116.62 81.66) (end 118.12 81.66) (width 0.25) (layer F.Cu) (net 10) (status 20))
 (segment (start 115.884999 80.924999) (end 116.62 81.66) (width 0.25) (layer F.Cu) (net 10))
 (segment (start 115.884999 70.805001) (end 115.884999 80.924999) (width 0.25) (layer F.Cu) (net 10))
 (segment (start 116.96 69.73) (end 115.884999 70.805001) (width 0.25) (layer F.Cu) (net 10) (status 10))
 (segment (start 134.366 75.438) (end 134.366 88.7095) (width 0.5) (layer B.Cu) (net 16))
 (segment (start 134.366 88.7095) (end 133.2865 89.789) (width 0.5) (layer B.Cu) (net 16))
 (segment (start 133.2865 89.789) (end 133.2865 89.789) (width 0.5) (layer B.Cu) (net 16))
 (via (at 133.2865 89.789) (size 0.8) (drill 0.4) (layers F.Cu B.Cu) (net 16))
 (segment (start 127.7874 77.0926) (end 126.72 78.16) (width 0.5) (layer F.Cu) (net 14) (status 20))
 (segment (start 127.7874 75.3488) (end 127.7874 77.0926) (width 0.5) (layer F.Cu) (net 14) (status 10))
 (segment (start 125.5268 77.3532) (end 124.72 78.16) (width 0.5) (layer F.Cu) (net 8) (status 20))
 (segment (start 125.5268 75.368) (end 125.5268 77.3532) (width 0.5) (layer F.Cu) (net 8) (status 10))
 (segment (start 119.869999 79.340001) (end 120.412998 79.883) (width 0.5) (layer F.Cu) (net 8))
 (segment (start 119.869999 74.560001) (end 119.869999 79.340001) (width 0.5) (layer F.Cu) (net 8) (status 10))
 (segment (start 120.07 74.36) (end 119.869999 74.560001) (width 0.5) (layer F.Cu) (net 8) (status 30))
 (segment (start 120.412998 79.883) (end 123.825 79.883) (width 0.5) (layer F.Cu) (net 8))
 (segment (start 124.72 78.988) (end 124.72 78.16) (width 0.5) (layer F.Cu) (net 8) (status 30))
 (segment (start 123.825 79.883) (end 124.72 78.988) (width 0.5) (layer F.Cu) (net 8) (status 20))
 (via (at 125.21 65.3) (size 0.8) (drill 0.4) (layers F.Cu B.Cu) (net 7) (status 30))
 (via (at 126.95 62.04) (size 0.8) (drill 0.4) (layers F.Cu B.Cu) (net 7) (status 30))
 (segment (start 126.95 62.04) (end 126.52 61.61) (width 0.5) (layer B.Cu) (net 7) (status 30))
 (segment (start 126.52 60.34) (end 126.6 60.26) (width 0.5) (layer B.Cu) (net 7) (status 30))
 (segment (start 126.52 61.61) (end 126.52 60.34) (width 0.5) (layer B.Cu) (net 7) (status 30))
 (segment (start 127.27 62.04) (end 128.8 60.51) (width 0.5) (layer B.Cu) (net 7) (status 30))
 (segment (start 126.95 62.04) (end 127.27 62.04) (width 0.5) (layer B.Cu) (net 7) (status 30))
 (segment (start 125.7808 63.0492) (end 126.82 62.01) (width 0.5) (layer B.Cu) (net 7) (status 30))
 (segment (start 125.7808 64.0842) (end 125.7808 63.0492) (width 0.5) (layer B.Cu) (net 7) (status 30))
 (segment (start 122.3 60.51) (end 128.8 60.51) (width 0.5) (layer F.Cu) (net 7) (status 30))
 (segment (start 132.679999 65.520001) (end 130.98 67.22) (width 0.5) (layer B.Cu) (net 17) (status 20))
 (segment (start 133.485001 65.520001) (end 132.679999 65.520001) (width 0.5) (layer B.Cu) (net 17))
 (segment (start 135.188 63.817002) (end 133.485001 65.520001) (width 0.5) (layer B.Cu) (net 17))
 (segment (start 135.188 60.69) (end 135.188 63.817002) (width 0.5) (layer B.Cu) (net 17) (status 10))
 (segment (start 130.048 76.832) (end 128.72 78.16) (width 0.5) (layer F.Cu) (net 15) (status 20))
 (segment (start 130.048 75.3488) (end 130.048 76.832) (width 0.5) (layer F.Cu) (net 15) (status 10))
 (segment (start 124.72 57.64) (end 124.7 57.66) (width 0.5) (layer B.Cu) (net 5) (status 30))
 (segment (start 124.72 55.66) (end 124.72 57.64) (width 0.5) (layer B.Cu) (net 5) (status 30))
 (via (at 124.7 57.66) (size 0.8) (drill 0.4) (layers F.Cu B.Cu) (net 5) (status 30))
 (segment (start 124.7 57.66) (end 124.940001 57.419999) (width 0.5) (layer F.Cu) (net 5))
 (segment (start 122.89844 57.66) (end 124.7 57.66) (width 0.25) (layer F.Cu) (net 5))
 (segment (start 120.69572 59.86272) (end 122.89844 57.66) (width 0.25) (layer F.Cu) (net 5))
 (segment (start 121.998718 62.02172) (end 120.69572 60.718722) (width 0.25) (layer F.Cu) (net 5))
 (segment (start 122.71248 62.02172) (end 121.998718 62.02172) (width 0.25) (layer F.Cu) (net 5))
 (segment (start 124.29236 76.58764) (end 124.29236 72.19696) (width 0.25) (layer F.Cu) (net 5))
 (segment (start 120.69572 60.718722) (end 120.69572 59.86272) (width 0.25) (layer F.Cu) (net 5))
 (segment (start 124.29236 72.19696) (end 126.07544 70.41388) (width 0.25) (layer F.Cu) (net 5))
 (segment (start 126.07544 70.41388) (end 126.07544 67.98564) (width 0.25) (layer F.Cu) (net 5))
 (segment (start 123.73864 65.64884) (end 123.73864 63.64224) (width 0.25) (layer F.Cu) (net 5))
 (segment (start 126.07544 67.98564) (end 123.73864 65.64884) (width 0.25) (layer F.Cu) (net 5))
 (segment (start 124.46 62.92088) (end 125.49124 62.92088) (width 0.25) (layer F.Cu) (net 5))
 (segment (start 123.73864 63.64224) (end 124.46 62.92088) (width 0.25) (layer F.Cu) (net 5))
 (segment (start 122.72 78.16) (end 124.29236 76.58764) (width 0.25) (layer F.Cu) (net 5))
 (segment (start 125.68428 62.72784) (end 125.68428 61.449278) (width 0.25) (layer F.Cu) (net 5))
 (segment (start 125.68428 61.449278) (end 125.316922 61.08192) (width 0.25) (layer F.Cu) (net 5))
 (segment (start 125.49124 62.92088) (end 125.68428 62.72784) (width 0.25) (layer F.Cu) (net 5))
 (segment (start 125.316922 61.08192) (end 123.65228 61.08192) (width 0.25) (layer F.Cu) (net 5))
 (segment (start 123.65228 61.08192) (end 122.71248 62.02172) (width 0.25) (layer F.Cu) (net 5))
 (segment (start 123.0376 71.8749) (end 125.0825 69.83) (width 0.5) (layer F.Cu) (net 19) (status 20))
 (segment (start 123.0376 73.0188) (end 123.0376 71.8749) (width 0.5) (layer F.Cu) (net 19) (status 10))
 (segment (start 123.0376 75.8424) (end 120.72 78.16) (width 0.5) (layer F.Cu) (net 13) (status 30))
 (segment (start 123.0376 75.4188) (end 123.0376 75.8424) (width 0.5) (layer F.Cu) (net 13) (status 30))
 (segment (start 131.41 60.495) (end 131.45 60.535) (width 0.5) (layer F.Cu) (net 20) (status 30))
 (segment (start 131.41 58.52) (end 131.41 60.495) (width 0.5) (layer F.Cu) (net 20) (status 30))
 (segment (start 123.13 58.69) (end 124.7 60.26) (width 0.5) (layer B.Cu) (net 6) (status 30))
 (segment (start 122.88 58.69) (end 123.13 58.69) (width 0.5) (layer B.Cu) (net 6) (status 30))
 (segment (start 122.88 56.59) (end 122.3 56.01) (width 0.5) (layer B.Cu) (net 6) (status 30))
 (segment (start 122.88 58.69) (end 122.88 56.59) (width 0.5) (layer B.Cu) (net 6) (status 30))
 (segment (start 128.8 56.01) (end 122.3 56.01) (width 0.5) (layer F.Cu) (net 6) (status 30))
 (segment (start 128.91 56.12) (end 128.8 56.01) (width 0.5) (layer F.Cu) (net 6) (status 30))
 (segment (start 131.41 56.12) (end 128.91 56.12) (width 0.5) (layer F.Cu) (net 6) (status 30))
 (via (at 132.821162 64.111162) (size 0.8) (drill 0.4) (layers F.Cu B.Cu) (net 18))
 (segment (start 129.59 66.25) (end 130.682324 66.25) (width 0.5) (layer F.Cu) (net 18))
 (segment (start 130.682324 66.25) (end 132.821162 64.111162) (width 0.5) (layer F.Cu) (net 18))
 (segment (start 130.98 61.354) (end 130.98 64.17) (width 0.5) (layer B.Cu) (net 12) (status 30))
 (segment (start 131.484 60.85) (end 130.98 61.354) (width 0.5) (layer B.Cu) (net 12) (status 30))
 (segment (start 128.91 64.53) (end 129.59 63.85) (width 0.5) (layer F.Cu) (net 12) (status 30))
 (segment (start 127.21 64.53) (end 128.91 64.53) (width 0.5) (layer F.Cu) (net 12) (status 30))
 (via (at 130.955824 64.915824) (size 0.8) (drill 0.4) (layers F.Cu B.Cu) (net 12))
 (segment (start 129.59 63.85) (end 129.89 63.85) (width 0.5) (layer F.Cu) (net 12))
 (segment (start 129.89 63.85) (end 130.955824 64.915824) (width 0.5) (layer F.Cu) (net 12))
 (segment (start 128.458011 58.170009) (end 125.774996 58.170009) (width 0.5) (layer F.Cu) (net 3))
 (via (at 125.774996 58.170009) (size 0.8) (drill 0.4) (layers F.Cu B.Cu) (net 3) (status 30))
 (segment (start 125.21 63.58) (end 127.728002 63.58) (width 0.5) (layer F.Cu) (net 3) (status 10))
 (segment (start 127.728002 63.58) (end 130.150001 61.158001) (width 0.5) (layer F.Cu) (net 3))
 (segment (start 130.150001 61.158001) (end 130.150001 59.861999) (width 0.5) (layer F.Cu) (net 3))
 (segment (start 130.150001 59.861999) (end 128.458011 58.170009) (width 0.5) (layer F.Cu) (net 3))
 (segment (start 134.8715 67.707) (end 134.8715 59.32682) (width 0.25) (layer F.Cu) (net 3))
 (segment (start 126.710004 57.235001) (end 125.774996 58.170009) (width 0.25) (layer F.Cu) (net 3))
 (segment (start 132.779681 57.235001) (end 126.710004 57.235001) (width 0.25) (layer F.Cu) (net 3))
 (segment (start 134.8715 59.32682) (end 132.779681 57.235001) (width 0.25) (layer F.Cu) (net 3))
 (segment (start 135.605 79.66) (end 133.32 79.66) (width 0.5) (layer F.Cu) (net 1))
 (segment (start 135.8265 79.4385) (end 135.605 79.66) (width 0.5) (layer F.Cu) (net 1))
 (segment (start 135.8265 71.612) (end 135.8265 79.4385) (width 0.5) (layer F.Cu) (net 1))
 (segment (start 133.9215 69.707) (end 135.8265 71.612) (width 0.5) (layer F.Cu) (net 1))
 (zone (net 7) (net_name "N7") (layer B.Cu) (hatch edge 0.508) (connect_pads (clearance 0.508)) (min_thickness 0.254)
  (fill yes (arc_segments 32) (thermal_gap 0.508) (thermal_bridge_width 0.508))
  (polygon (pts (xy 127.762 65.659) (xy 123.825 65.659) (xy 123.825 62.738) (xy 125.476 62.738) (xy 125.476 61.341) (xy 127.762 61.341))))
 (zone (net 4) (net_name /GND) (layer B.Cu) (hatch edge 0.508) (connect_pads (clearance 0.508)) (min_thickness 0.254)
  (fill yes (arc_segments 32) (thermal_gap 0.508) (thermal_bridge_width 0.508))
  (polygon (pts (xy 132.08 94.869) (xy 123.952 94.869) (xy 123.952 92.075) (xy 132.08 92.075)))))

